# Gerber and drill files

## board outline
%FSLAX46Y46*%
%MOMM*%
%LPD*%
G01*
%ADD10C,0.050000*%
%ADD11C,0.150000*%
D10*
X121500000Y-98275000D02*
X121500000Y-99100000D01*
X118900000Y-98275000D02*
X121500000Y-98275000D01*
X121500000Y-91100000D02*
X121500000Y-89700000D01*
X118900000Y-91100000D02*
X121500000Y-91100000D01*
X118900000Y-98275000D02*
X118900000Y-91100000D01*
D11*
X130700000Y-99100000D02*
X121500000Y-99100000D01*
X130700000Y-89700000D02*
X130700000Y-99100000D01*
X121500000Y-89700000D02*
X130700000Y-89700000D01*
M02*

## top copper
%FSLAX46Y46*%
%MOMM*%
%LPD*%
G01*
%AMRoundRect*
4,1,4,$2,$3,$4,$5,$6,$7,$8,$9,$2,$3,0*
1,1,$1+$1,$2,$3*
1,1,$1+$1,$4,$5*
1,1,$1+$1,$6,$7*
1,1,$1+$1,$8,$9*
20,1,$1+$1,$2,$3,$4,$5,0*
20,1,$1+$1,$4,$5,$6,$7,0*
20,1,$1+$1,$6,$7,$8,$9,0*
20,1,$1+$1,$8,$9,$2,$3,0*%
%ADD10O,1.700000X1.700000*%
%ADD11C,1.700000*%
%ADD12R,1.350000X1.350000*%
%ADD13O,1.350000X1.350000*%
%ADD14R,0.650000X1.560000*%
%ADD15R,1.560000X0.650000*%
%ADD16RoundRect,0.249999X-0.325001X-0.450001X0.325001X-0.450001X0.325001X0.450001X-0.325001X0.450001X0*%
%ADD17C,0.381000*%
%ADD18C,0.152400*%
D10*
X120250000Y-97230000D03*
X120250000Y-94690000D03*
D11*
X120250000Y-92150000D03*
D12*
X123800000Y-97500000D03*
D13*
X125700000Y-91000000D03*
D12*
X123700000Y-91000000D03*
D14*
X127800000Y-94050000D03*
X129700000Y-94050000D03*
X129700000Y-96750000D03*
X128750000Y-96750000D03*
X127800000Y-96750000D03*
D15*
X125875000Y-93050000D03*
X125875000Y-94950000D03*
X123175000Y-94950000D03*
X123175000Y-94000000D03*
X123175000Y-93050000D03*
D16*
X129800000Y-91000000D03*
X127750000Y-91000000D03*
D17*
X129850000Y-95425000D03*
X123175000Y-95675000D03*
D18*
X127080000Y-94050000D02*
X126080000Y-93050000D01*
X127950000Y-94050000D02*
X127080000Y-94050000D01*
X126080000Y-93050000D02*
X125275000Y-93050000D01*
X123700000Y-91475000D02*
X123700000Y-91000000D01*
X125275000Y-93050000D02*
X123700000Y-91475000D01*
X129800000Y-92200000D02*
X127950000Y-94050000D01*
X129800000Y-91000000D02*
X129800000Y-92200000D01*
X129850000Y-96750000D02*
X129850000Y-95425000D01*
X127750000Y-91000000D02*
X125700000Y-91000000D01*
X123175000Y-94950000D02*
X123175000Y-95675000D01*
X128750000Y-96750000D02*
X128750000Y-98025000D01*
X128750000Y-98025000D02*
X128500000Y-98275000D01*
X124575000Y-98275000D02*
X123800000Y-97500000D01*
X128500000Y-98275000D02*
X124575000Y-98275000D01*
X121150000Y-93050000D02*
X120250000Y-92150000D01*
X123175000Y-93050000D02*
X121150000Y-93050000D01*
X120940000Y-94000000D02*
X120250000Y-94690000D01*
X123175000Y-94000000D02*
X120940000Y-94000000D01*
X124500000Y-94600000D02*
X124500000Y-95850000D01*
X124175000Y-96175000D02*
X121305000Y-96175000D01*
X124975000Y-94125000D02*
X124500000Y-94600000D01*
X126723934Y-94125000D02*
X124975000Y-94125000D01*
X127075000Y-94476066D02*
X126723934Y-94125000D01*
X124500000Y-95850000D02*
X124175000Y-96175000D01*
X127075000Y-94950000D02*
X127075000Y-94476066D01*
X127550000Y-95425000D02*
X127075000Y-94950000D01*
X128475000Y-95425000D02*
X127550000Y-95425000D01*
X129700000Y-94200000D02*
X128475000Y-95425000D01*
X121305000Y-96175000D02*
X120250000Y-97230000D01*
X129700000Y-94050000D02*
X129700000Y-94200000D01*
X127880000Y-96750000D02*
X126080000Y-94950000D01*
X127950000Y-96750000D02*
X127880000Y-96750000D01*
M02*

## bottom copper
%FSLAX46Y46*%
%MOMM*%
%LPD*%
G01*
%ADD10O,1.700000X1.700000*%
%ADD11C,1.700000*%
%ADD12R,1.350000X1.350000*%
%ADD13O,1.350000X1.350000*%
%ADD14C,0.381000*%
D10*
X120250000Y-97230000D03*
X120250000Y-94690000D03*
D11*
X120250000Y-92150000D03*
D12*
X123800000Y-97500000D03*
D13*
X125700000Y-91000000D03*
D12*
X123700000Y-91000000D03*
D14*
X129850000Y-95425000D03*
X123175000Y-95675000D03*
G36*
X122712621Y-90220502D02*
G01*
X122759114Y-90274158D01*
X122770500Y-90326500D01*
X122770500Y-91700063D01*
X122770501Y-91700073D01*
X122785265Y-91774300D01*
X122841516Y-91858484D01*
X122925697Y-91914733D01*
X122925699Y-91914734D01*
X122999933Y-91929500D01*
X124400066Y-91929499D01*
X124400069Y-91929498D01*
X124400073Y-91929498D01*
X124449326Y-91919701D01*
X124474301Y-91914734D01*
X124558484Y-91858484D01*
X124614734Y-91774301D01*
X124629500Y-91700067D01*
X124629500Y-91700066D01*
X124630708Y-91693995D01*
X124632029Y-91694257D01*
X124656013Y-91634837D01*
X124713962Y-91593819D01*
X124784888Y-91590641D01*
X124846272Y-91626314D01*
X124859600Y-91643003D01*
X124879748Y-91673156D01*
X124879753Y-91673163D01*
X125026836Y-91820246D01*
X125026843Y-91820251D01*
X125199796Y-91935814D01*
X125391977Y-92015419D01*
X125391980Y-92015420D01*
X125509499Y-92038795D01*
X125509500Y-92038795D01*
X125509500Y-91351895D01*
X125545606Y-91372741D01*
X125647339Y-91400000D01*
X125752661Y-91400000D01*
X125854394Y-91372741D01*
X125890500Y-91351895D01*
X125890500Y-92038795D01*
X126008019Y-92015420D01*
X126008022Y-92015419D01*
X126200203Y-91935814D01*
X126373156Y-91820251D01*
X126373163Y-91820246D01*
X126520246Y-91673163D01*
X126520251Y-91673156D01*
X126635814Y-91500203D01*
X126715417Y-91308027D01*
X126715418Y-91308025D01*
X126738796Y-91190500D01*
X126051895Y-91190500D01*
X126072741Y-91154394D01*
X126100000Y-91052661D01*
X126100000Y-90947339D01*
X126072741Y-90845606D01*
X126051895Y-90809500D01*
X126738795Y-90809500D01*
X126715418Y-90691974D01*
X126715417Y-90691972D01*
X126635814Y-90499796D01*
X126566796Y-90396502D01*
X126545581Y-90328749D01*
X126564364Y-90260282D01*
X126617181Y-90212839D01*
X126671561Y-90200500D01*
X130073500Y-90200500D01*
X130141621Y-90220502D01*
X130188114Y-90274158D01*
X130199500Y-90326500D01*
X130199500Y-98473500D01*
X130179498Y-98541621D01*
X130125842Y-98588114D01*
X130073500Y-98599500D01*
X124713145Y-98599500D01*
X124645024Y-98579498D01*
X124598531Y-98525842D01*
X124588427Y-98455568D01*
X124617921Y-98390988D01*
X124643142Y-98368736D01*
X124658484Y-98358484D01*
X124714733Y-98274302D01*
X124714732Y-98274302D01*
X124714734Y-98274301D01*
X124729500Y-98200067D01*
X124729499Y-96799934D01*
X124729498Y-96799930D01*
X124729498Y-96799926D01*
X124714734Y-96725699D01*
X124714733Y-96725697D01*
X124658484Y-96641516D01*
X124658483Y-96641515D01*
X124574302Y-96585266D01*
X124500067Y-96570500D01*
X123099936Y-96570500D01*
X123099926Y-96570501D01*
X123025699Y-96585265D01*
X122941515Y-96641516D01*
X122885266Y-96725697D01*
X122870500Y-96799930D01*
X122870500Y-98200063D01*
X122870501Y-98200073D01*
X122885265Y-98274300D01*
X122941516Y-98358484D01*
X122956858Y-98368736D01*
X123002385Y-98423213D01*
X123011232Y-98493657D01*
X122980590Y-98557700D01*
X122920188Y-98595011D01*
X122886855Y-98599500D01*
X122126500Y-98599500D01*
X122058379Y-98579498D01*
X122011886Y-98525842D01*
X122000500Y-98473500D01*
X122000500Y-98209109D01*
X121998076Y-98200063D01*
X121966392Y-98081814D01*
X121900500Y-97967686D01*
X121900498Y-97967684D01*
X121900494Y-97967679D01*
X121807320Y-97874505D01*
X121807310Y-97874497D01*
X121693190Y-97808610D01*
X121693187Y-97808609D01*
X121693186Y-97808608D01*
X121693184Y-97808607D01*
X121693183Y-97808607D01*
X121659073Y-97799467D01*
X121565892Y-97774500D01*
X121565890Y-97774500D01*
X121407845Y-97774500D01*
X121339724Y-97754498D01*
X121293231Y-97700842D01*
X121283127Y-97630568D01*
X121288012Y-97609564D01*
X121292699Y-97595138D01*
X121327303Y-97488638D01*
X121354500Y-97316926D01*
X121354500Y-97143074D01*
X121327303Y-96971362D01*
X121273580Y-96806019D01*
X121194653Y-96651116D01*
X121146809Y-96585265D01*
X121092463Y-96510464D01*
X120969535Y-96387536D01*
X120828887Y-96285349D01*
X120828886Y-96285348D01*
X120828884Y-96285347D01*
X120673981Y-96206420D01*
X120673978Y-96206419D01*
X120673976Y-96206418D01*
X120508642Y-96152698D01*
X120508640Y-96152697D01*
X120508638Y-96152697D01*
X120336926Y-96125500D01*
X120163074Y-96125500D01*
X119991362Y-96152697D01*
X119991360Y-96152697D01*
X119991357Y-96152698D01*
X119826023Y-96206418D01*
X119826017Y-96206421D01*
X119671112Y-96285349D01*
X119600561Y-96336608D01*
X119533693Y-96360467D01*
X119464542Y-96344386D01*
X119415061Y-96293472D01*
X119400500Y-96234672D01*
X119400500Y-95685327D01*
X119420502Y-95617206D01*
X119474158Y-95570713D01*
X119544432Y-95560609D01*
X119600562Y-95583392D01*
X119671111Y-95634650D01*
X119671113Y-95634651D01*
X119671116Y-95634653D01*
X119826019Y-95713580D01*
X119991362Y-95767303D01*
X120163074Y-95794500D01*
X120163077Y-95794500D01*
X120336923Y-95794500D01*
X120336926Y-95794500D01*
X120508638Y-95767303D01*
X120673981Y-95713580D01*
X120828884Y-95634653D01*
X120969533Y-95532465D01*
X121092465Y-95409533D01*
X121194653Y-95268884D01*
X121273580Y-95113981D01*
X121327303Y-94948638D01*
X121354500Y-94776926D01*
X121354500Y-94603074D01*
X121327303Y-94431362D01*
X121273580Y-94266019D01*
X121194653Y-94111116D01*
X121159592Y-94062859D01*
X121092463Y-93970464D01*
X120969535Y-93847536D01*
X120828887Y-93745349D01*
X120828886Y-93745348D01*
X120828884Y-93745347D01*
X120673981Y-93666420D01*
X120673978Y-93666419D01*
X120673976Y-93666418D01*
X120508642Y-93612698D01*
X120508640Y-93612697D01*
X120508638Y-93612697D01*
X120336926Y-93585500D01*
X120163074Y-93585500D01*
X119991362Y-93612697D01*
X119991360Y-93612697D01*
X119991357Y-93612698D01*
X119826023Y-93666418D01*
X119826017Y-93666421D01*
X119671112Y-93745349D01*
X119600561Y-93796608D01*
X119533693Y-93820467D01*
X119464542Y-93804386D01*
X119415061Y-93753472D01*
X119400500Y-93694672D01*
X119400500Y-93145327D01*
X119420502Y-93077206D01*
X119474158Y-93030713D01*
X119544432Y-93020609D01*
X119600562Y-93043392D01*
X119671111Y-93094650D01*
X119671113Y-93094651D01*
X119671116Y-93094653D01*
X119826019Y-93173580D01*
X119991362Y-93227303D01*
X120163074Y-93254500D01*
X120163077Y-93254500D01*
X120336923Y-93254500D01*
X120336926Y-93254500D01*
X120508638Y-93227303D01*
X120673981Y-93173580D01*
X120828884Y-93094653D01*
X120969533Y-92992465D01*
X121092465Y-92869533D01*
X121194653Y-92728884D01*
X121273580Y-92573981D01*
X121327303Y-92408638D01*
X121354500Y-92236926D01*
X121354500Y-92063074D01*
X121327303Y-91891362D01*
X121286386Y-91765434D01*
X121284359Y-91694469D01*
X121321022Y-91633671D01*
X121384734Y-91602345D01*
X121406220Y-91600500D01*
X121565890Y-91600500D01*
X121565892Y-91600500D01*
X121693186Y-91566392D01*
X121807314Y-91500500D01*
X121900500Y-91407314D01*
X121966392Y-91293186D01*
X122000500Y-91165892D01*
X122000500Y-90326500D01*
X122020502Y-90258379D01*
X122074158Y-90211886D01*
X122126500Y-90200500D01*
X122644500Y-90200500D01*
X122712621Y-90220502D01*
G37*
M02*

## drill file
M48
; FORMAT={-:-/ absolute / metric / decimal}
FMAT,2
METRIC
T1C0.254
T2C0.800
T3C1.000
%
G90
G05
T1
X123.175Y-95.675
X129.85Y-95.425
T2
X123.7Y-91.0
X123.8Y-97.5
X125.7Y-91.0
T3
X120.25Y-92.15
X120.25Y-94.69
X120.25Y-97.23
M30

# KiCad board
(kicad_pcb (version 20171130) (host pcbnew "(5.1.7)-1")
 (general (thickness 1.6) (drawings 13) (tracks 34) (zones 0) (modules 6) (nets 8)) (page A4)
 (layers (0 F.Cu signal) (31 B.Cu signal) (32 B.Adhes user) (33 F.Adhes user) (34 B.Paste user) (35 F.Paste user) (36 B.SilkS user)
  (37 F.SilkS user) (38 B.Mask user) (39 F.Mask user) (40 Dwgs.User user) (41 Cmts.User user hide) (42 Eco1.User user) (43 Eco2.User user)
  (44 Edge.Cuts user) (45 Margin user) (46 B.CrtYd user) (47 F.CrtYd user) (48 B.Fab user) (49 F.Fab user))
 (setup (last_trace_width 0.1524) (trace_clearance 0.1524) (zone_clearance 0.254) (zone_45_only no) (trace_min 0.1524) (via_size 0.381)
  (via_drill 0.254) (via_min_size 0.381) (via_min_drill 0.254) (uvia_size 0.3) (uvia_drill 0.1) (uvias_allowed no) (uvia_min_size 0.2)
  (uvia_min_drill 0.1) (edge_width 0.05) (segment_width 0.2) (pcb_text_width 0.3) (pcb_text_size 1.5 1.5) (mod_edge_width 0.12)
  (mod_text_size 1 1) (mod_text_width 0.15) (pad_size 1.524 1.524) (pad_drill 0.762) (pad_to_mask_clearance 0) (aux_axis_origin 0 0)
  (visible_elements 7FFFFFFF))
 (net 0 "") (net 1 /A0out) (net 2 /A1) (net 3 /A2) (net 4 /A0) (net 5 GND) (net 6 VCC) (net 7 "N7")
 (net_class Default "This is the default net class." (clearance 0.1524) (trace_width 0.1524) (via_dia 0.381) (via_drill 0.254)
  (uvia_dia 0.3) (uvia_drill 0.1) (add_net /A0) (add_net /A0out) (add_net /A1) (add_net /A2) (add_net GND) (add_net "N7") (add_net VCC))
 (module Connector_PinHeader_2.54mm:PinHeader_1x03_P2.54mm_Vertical (layer F.Cu) (at 120.25 92.15)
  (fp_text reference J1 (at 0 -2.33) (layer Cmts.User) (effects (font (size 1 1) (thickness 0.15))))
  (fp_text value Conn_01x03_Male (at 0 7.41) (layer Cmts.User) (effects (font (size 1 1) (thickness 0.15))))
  (pad 3 thru_hole oval (at 0 5.08) (size 1.7 1.7) (drill 1) (layers *.Cu *.Mask) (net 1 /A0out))
  (pad 2 thru_hole oval (at 0 2.54) (size 1.7 1.7) (drill 1) (layers *.Cu *.Mask) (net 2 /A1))
  (pad 1 thru_hole circle (at 0 0) (size 1.7 1.7) (drill 1) (layers *.Cu *.Mask) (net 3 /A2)))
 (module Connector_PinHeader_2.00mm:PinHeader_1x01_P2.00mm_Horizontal (layer F.Cu) (at 123.8 97.5)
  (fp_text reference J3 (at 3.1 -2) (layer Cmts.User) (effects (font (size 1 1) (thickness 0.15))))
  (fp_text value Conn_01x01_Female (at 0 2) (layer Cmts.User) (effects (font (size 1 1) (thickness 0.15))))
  (pad 1 thru_hole rect (at 0 0) (size 1.35 1.35) (drill 0.8) (layers *.Cu *.Mask) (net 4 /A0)))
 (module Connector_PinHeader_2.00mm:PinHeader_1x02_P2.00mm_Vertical (layer F.Cu) (at 123.7 91 90)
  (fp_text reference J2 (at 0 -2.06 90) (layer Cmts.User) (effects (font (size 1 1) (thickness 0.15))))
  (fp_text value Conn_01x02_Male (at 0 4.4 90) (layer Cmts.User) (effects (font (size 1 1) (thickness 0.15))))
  (pad 2 thru_hole oval (at 0 2 90) (size 1.35 1.35) (drill 0.8) (layers *.Cu *.Mask) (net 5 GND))
  (pad 1 thru_hole rect (at 0 0 90) (size 1.35 1.35) (drill 0.8) (layers *.Cu *.Mask) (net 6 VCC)))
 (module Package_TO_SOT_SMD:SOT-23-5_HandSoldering (layer F.Cu) (at 128.75 95.4 90)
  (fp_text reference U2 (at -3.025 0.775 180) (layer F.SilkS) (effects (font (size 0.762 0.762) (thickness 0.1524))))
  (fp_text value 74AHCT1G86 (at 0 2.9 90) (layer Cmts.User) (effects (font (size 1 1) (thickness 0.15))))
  (pad 5 smd rect (at 1.35 -0.95 90) (size 1.56 0.65) (layers F.Cu F.Paste F.Mask) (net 6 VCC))
  (pad 4 smd rect (at 1.35 0.95 90) (size 1.56 0.65) (layers F.Cu F.Paste F.Mask) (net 1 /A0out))
  (pad 3 smd rect (at -1.35 0.95 90) (size 1.56 0.65) (layers F.Cu F.Paste F.Mask) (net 5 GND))
  (pad 2 smd rect (at -1.35 0 90) (size 1.56 0.65) (layers F.Cu F.Paste F.Mask) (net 4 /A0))
  (pad 1 smd rect (at -1.35 -0.95 90) (size 1.56 0.65) (layers F.Cu F.Paste F.Mask) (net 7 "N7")))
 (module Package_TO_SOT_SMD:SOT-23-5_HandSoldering (layer F.Cu) (at 124.525 94)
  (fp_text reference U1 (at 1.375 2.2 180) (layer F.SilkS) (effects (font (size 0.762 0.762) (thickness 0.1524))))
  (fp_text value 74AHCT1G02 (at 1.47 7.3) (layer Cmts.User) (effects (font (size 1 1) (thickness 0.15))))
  (pad 5 smd rect (at 1.35 -0.95) (size 1.56 0.65) (layers F.Cu F.Paste F.Mask) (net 6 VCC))
  (pad 4 smd rect (at 1.35 0.95) (size 1.56 0.65) (layers F.Cu F.Paste F.Mask) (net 7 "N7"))
  (pad 3 smd rect (at -1.35 0.95) (size 1.56 0.65) (layers F.Cu F.Paste F.Mask) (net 5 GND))
  (pad 2 smd rect (at -1.35 0) (size 1.56 0.65) (layers F.Cu F.Paste F.Mask) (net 2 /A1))
  (pad 1 smd rect (at -1.35 -0.95) (size 1.56 0.65) (layers F.Cu F.Paste F.Mask) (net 3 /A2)))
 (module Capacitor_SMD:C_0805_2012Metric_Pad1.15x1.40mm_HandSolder (layer F.Cu) (at 128.775 91)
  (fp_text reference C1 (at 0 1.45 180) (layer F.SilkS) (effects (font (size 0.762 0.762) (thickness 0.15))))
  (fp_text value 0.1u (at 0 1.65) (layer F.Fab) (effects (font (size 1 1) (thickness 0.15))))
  (pad 2 smd roundrect (at 1.025 0) (size 1.15 1.4) (layers F.Cu F.Paste F.Mask) (roundrect_rratio 0.2173904347826087) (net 6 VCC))
  (pad 1 smd roundrect (at -1.025 0) (size 1.15 1.4) (layers F.Cu F.Paste F.Mask) (roundrect_rratio 0.2173904347826087) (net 5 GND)))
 (gr_line (start 121.5 98.275) (end 121.5 99.1) (layer Edge.Cuts) (width 0.05))
 (gr_line (start 118.9 98.275) (end 121.5 98.275) (layer Edge.Cuts) (width 0.05))
 (gr_line (start 121.5 91.1) (end 121.5 89.7) (layer Edge.Cuts) (width 0.05))
 (gr_line (start 118.9 91.1) (end 121.5 91.1) (layer Edge.Cuts) (width 0.05))
 (gr_line (start 118.9 98.275) (end 118.9 91.1) (layer Edge.Cuts) (width 0.05))
 (gr_line (start 130.7 99.1) (end 121.5 99.1) (layer Edge.Cuts) (width 0.15))
 (gr_line (start 130.7 89.7) (end 130.7 99.1) (layer Edge.Cuts) (width 0.15))
 (gr_line (start 121.5 89.7) (end 130.7 89.7) (layer Edge.Cuts) (width 0.15))
 (segment (start 127.08 94.05) (end 126.08 93.05) (width 0.1524) (layer F.Cu) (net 6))
 (segment (start 127.95 94.05) (end 127.08 94.05) (width 0.1524) (layer F.Cu) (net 6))
 (segment (start 126.08 93.05) (end 125.275 93.05) (width 0.1524) (layer F.Cu) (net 6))
 (segment (start 123.7 91.475) (end 123.7 91) (width 0.1524) (layer F.Cu) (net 6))
 (segment (start 125.275 93.05) (end 123.7 91.475) (width 0.1524) (layer F.Cu) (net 6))
 (segment (start 129.8 92.2) (end 127.95 94.05) (width 0.1524) (layer F.Cu) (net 6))
 (segment (start 129.8 91) (end 129.8 92.2) (width 0.1524) (layer F.Cu) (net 6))
 (via (at 129.85 95.425) (size 0.381) (drill 0.254) (layers F.Cu B.Cu) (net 5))
 (segment (start 129.85 96.75) (end 129.85 95.425) (width 0.1524) (layer F.Cu) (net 5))
 (segment (start 127.75 91) (end 125.7 91) (width 0.1524) (layer F.Cu) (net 5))
 (via (at 123.175 95.675) (size 0.381) (drill 0.254) (layers F.Cu B.Cu) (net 5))
 (segment (start 123.175 94.95) (end 123.175 95.675) (width 0.1524) (layer F.Cu) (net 5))
 (segment (start 128.75 96.75) (end 128.75 98.025) (width 0.1524) (layer F.Cu) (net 4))
 (segment (start 128.75 98.025) (end 128.5 98.275) (width 0.1524) (layer F.Cu) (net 4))
 (segment (start 124.575 98.275) (end 123.8 97.5) (width 0.1524) (layer F.Cu) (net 4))
 (segment (start 128.5 98.275) (end 124.575 98.275) (width 0.1524) (layer F.Cu) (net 4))
 (segment (start 121.15 93.05) (end 120.25 92.15) (width 0.1524) (layer F.Cu) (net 3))
 (segment (start 123.175 93.05) (end 121.15 93.05) (width 0.1524) (layer F.Cu) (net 3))
 (segment (start 120.94 94) (end 120.25 94.69) (width 0.1524) (layer F.Cu) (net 2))
 (segment (start 123.175 94) (end 120.94 94) (width 0.1524) (layer F.Cu) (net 2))
 (segment (start 124.5 94.6) (end 124.5 95.85) (width 0.1524) (layer F.Cu) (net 1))
 (segment (start 124.175 96.175) (end 121.305 96.175) (width 0.1524) (layer F.Cu) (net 1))
 (segment (start 124.975 94.125) (end 124.5 94.6) (width 0.1524) (layer F.Cu) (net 1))
 (segment (start 126.723934 94.125) (end 124.975 94.125) (width 0.1524) (layer F.Cu) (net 1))
 (segment (start 127.075 94.476066) (end 126.723934 94.125) (width 0.1524) (layer F.Cu) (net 1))
 (segment (start 124.5 95.85) (end 124.175 96.175) (width 0.1524) (layer F.Cu) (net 1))
 (segment (start 127.075 94.95) (end 127.075 94.476066) (width 0.1524) (layer F.Cu) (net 1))
 (segment (start 127.55 95.425) (end 127.075 94.95) (width 0.1524) (layer F.Cu) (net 1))
 (segment (start 128.475 95.425) (end 127.55 95.425) (width 0.1524) (layer F.Cu) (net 1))
 (segment (start 129.7 94.2) (end 128.475 95.425) (width 0.1524) (layer F.Cu) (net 1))
 (segment (start 121.305 96.175) (end 120.25 97.23) (width 0.1524) (layer F.Cu) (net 1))
 (segment (start 129.7 94.05) (end 129.7 94.2) (width 0.1524) (layer F.Cu) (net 1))
 (segment (start 127.88 96.75) (end 126.08 94.95) (width 0.1524) (layer F.Cu) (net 7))
 (segment (start 127.95 96.75) (end 127.88 96.75) (width 0.1524) (layer F.Cu) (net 7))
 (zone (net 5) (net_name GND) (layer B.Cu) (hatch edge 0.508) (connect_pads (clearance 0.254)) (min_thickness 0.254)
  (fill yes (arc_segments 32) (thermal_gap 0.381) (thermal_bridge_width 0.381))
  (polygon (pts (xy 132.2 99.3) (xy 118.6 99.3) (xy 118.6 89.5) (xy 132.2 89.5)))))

